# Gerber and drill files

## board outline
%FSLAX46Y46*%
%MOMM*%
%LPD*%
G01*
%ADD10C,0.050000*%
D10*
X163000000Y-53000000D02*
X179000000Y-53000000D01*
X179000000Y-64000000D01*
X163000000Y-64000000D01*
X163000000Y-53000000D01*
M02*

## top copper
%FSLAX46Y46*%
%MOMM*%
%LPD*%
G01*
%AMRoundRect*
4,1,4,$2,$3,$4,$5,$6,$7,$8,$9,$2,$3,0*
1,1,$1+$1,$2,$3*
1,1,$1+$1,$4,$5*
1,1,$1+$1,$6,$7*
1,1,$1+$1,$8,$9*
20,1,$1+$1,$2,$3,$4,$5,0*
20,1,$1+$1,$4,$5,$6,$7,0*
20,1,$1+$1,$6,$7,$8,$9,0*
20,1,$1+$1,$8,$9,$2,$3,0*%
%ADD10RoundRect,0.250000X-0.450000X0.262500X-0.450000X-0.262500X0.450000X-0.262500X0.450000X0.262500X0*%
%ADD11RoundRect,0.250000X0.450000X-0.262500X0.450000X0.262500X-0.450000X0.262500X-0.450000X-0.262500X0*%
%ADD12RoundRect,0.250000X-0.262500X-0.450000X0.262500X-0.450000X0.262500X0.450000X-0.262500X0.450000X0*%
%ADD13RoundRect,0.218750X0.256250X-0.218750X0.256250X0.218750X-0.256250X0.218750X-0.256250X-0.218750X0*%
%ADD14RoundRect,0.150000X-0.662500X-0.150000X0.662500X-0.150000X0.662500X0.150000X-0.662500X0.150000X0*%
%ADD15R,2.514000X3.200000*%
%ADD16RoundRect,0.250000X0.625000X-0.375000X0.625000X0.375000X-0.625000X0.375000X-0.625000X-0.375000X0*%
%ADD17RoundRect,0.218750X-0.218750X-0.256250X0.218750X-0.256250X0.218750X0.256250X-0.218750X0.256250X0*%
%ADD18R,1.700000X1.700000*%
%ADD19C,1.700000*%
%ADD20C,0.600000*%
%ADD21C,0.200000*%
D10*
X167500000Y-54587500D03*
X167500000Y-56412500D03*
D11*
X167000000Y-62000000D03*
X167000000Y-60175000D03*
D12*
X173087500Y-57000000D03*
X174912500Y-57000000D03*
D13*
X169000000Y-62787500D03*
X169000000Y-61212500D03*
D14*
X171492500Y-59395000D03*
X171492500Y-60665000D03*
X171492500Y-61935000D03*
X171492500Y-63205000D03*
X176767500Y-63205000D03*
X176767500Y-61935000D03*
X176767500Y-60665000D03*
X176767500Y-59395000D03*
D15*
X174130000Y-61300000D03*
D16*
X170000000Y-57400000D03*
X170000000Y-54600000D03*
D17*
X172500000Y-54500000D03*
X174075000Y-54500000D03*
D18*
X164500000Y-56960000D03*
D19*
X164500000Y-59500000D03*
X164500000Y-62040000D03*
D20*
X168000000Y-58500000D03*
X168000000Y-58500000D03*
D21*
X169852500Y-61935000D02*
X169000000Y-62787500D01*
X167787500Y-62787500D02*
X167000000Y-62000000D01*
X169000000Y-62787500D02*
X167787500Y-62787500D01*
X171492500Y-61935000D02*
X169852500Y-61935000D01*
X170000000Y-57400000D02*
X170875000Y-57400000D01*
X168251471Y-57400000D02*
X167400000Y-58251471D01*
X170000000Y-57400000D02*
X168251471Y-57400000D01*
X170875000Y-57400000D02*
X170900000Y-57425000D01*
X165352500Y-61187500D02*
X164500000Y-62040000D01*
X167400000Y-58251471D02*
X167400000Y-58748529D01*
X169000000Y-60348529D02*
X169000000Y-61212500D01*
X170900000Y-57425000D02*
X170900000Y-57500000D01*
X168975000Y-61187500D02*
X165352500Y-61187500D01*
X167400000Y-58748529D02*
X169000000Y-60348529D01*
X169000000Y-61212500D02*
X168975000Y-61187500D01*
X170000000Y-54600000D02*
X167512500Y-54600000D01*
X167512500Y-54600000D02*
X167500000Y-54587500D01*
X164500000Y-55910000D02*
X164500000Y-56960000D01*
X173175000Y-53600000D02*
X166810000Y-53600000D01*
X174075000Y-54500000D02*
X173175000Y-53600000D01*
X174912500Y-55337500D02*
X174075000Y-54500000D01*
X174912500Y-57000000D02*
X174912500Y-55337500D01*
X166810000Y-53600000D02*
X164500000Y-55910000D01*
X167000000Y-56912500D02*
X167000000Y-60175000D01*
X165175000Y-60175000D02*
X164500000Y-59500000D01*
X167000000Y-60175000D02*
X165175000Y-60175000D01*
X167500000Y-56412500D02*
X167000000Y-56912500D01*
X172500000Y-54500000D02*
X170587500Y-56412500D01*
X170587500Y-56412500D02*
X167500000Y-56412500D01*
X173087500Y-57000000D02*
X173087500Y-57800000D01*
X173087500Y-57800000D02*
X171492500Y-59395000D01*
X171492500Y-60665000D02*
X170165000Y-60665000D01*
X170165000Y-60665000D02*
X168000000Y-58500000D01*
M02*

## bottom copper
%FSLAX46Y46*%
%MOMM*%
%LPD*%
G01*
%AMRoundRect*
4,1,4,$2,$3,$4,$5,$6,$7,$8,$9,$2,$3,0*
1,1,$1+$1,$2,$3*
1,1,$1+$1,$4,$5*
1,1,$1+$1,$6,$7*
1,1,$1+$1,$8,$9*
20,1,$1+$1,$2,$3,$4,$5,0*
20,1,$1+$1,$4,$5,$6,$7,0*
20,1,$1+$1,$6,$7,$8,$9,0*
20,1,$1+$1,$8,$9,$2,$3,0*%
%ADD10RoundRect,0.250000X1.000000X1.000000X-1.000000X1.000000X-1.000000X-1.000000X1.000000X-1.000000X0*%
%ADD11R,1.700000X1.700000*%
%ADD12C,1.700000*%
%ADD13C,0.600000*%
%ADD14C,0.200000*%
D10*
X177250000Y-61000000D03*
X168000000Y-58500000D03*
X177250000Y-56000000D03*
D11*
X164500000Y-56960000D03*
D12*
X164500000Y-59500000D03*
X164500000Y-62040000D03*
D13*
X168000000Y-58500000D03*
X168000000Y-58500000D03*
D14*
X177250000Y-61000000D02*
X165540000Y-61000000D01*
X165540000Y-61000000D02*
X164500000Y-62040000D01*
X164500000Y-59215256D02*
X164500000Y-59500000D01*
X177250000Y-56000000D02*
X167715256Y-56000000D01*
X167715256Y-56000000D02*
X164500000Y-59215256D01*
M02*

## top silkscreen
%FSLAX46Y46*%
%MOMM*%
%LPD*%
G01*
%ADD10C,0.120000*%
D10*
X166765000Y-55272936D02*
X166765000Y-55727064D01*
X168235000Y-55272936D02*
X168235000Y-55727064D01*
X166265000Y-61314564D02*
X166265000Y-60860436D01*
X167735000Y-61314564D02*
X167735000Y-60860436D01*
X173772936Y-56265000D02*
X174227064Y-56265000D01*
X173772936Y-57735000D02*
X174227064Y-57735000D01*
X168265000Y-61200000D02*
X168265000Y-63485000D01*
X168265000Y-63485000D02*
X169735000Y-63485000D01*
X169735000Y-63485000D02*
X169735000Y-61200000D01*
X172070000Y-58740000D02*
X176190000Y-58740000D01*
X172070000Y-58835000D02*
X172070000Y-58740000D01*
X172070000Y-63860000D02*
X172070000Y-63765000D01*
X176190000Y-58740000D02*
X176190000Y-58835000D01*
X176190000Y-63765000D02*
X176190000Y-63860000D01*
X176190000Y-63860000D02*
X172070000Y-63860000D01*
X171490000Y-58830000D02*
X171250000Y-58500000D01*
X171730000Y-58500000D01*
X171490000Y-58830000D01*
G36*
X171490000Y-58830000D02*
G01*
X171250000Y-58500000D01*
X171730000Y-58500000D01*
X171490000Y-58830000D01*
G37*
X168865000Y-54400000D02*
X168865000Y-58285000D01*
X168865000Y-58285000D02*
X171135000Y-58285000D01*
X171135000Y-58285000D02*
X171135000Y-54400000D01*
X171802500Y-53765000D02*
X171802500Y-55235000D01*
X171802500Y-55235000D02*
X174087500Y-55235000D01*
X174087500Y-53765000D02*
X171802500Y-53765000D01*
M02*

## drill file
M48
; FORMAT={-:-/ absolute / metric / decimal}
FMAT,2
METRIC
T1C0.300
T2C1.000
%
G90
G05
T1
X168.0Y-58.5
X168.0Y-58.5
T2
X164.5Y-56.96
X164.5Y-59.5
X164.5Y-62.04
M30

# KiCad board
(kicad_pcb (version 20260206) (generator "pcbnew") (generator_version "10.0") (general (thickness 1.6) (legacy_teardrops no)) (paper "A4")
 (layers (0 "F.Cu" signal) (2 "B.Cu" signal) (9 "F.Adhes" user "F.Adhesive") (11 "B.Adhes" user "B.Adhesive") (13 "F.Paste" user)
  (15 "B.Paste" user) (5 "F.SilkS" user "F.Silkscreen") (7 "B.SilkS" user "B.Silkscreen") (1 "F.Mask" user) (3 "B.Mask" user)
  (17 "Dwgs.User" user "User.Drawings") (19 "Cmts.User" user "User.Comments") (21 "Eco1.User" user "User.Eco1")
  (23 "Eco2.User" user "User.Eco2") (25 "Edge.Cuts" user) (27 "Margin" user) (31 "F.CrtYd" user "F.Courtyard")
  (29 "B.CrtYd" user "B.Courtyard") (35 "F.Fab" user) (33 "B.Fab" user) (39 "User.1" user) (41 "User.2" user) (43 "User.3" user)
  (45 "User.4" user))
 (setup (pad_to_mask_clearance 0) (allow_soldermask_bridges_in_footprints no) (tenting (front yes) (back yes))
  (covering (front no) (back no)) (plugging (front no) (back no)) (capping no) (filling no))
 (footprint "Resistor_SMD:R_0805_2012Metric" (layer "F.Cu") (at 167.5 55.5 -90)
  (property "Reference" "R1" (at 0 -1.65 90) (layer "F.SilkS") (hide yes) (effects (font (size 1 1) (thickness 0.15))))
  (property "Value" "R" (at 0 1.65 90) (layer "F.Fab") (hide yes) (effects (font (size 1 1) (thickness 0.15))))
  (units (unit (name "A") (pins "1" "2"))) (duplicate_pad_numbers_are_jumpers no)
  (fp_line (start -0.227064 0.735) (end 0.227064 0.735) (stroke (width 0.12) (type solid)) (layer "F.SilkS"))
  (fp_line (start -0.227064 -0.735) (end 0.227064 -0.735) (stroke (width 0.12) (type solid)) (layer "F.SilkS"))
  (pad "1" smd roundrect (at -0.9125 0 270) (size 1.025 1.4) (layers "F.Cu" "F.Mask" "F.Paste") (roundrect_rratio 0.243902)
   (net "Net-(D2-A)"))
  (pad "2" smd roundrect (at 0.9125 0 270) (size 1.025 1.4) (layers "F.Cu" "F.Mask" "F.Paste") (roundrect_rratio 0.243902) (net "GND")))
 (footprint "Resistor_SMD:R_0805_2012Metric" (layer "F.Cu") (at 167 61.0875 90)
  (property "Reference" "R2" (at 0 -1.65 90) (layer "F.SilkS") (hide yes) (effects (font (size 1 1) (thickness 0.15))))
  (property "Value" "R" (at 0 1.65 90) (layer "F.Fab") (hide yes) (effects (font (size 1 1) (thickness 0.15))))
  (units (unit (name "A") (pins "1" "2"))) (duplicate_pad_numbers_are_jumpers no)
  (fp_line (start -0.227064 -0.735) (end 0.227064 -0.735) (stroke (width 0.12) (type solid)) (layer "F.SilkS"))
  (fp_line (start -0.227064 0.735) (end 0.227064 0.735) (stroke (width 0.12) (type solid)) (layer "F.SilkS"))
  (pad "1" smd roundrect (at -0.9125 0 90) (size 1.025 1.4) (layers "F.Cu" "F.Mask" "F.Paste") (roundrect_rratio 0.243902)
   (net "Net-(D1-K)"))
  (pad "2" smd roundrect (at 0.9125 0 90) (size 1.025 1.4) (layers "F.Cu" "F.Mask" "F.Paste") (roundrect_rratio 0.243902) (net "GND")))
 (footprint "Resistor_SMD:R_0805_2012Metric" (layer "F.Cu") (at 174 57)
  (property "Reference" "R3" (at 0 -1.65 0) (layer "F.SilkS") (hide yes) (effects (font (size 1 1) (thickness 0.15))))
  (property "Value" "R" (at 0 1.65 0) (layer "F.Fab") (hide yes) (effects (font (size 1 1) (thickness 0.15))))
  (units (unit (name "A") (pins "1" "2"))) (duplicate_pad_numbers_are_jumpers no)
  (fp_line (start -0.227064 -0.735) (end 0.227064 -0.735) (stroke (width 0.12) (type solid)) (layer "F.SilkS"))
  (fp_line (start -0.227064 0.735) (end 0.227064 0.735) (stroke (width 0.12) (type solid)) (layer "F.SilkS"))
  (pad "1" smd roundrect (at -0.9125 0) (size 1.025 1.4) (layers "F.Cu" "F.Mask" "F.Paste") (roundrect_rratio 0.243902)
   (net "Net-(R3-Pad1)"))
  (pad "2" smd roundrect (at 0.9125 0) (size 1.025 1.4) (layers "F.Cu" "F.Mask" "F.Paste") (roundrect_rratio 0.243902) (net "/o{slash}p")))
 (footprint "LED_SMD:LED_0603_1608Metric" (layer "F.Cu") (at 169 62 90)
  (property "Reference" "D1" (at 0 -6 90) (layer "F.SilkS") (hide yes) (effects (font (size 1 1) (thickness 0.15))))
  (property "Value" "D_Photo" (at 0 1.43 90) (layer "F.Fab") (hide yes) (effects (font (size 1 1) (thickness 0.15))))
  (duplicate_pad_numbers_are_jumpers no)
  (fp_line (start 0.8 -0.735) (end -1.485 -0.735) (stroke (width 0.12) (type solid)) (layer "F.SilkS"))
  (fp_line (start -1.485 -0.735) (end -1.485 0.735) (stroke (width 0.12) (type solid)) (layer "F.SilkS"))
  (fp_line (start -1.485 0.735) (end 0.8 0.735) (stroke (width 0.12) (type solid)) (layer "F.SilkS"))
  (pad "1" smd roundrect (at -0.7875 0 90) (size 0.875 0.95) (layers "F.Cu" "F.Mask" "F.Paste") (roundrect_rratio 0.25) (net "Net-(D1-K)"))
  (pad "2" smd roundrect (at 0.7875 0 90) (size 0.875 0.95) (layers "F.Cu" "F.Mask" "F.Paste") (roundrect_rratio 0.25) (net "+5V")))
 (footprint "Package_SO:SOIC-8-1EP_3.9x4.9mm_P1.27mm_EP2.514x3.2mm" (layer "F.Cu") (at 174.13 61.3)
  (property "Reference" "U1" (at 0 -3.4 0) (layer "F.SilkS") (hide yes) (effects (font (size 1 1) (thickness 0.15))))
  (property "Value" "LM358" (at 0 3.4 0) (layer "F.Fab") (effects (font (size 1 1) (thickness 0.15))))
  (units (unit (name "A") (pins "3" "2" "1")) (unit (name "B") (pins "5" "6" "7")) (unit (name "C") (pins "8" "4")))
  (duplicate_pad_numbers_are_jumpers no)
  (fp_line (start -2.06 -2.56) (end 2.06 -2.56) (stroke (width 0.12) (type solid)) (layer "F.SilkS"))
  (fp_line (start -2.06 -2.465) (end -2.06 -2.56) (stroke (width 0.12) (type solid)) (layer "F.SilkS"))
  (fp_line (start -2.06 2.56) (end -2.06 2.465) (stroke (width 0.12) (type solid)) (layer "F.SilkS"))
  (fp_line (start 2.06 -2.56) (end 2.06 -2.465) (stroke (width 0.12) (type solid)) (layer "F.SilkS"))
  (fp_line (start 2.06 2.465) (end 2.06 2.56) (stroke (width 0.12) (type solid)) (layer "F.SilkS"))
  (fp_line (start 2.06 2.56) (end -2.06 2.56) (stroke (width 0.12) (type solid)) (layer "F.SilkS"))
  (fp_poly (pts (xy -2.64 -2.47) (xy -2.88 -2.8) (xy -2.4 -2.8)) (stroke (width 0.12) (type solid)) (fill yes) (layer "F.SilkS"))
  (pad "" smd roundrect (at -0.63 -0.8) (size 1.01 1.29) (layers "F.Paste") (roundrect_rratio 0.247525))
  (pad "" smd roundrect (at -0.63 0.8) (size 1.01 1.29) (layers "F.Paste") (roundrect_rratio 0.247525))
  (pad "" smd roundrect (at 0.63 -0.8) (size 1.01 1.29) (layers "F.Paste") (roundrect_rratio 0.247525))
  (pad "" smd roundrect (at 0.63 0.8) (size 1.01 1.29) (layers "F.Paste") (roundrect_rratio 0.247525))
  (pad "1" smd roundrect (at -2.6375 -1.905) (size 1.625 0.6) (layers "F.Cu" "F.Mask" "F.Paste") (roundrect_rratio 0.25)
   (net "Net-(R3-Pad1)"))
  (pad "2" smd roundrect (at -2.6375 -0.635) (size 1.625 0.6) (layers "F.Cu" "F.Mask" "F.Paste") (roundrect_rratio 0.25) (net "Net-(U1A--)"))
  (pad "3" smd roundrect (at -2.6375 0.635) (size 1.625 0.6) (layers "F.Cu" "F.Mask" "F.Paste") (roundrect_rratio 0.25) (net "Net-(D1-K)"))
  (pad "4" smd roundrect (at -2.6375 1.905) (size 1.625 0.6) (layers "F.Cu" "F.Mask" "F.Paste") (roundrect_rratio 0.25))
  (pad "5" smd roundrect (at 2.6375 1.905) (size 1.625 0.6) (layers "F.Cu" "F.Mask" "F.Paste") (roundrect_rratio 0.25))
  (pad "6" smd roundrect (at 2.6375 0.635) (size 1.625 0.6) (layers "F.Cu" "F.Mask" "F.Paste") (roundrect_rratio 0.25))
  (pad "7" smd roundrect (at 2.6375 -0.635) (size 1.625 0.6) (layers "F.Cu" "F.Mask" "F.Paste") (roundrect_rratio 0.25))
  (pad "8" smd roundrect (at 2.6375 -1.905) (size 1.625 0.6) (layers "F.Cu" "F.Mask" "F.Paste") (roundrect_rratio 0.25))
  (pad "9" smd rect (at 0 0) (size 2.514 3.2) (layers "F.Cu" "F.Mask") (zone_connect 2)))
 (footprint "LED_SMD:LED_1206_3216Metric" (layer "F.Cu") (at 170 56 90)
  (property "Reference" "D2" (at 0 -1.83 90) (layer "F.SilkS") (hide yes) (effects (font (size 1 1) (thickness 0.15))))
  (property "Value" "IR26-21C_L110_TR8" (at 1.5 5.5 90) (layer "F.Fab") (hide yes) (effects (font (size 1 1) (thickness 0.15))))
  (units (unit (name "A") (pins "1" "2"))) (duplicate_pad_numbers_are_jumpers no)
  (fp_line (start 1.6 -1.135) (end -2.285 -1.135) (stroke (width 0.12) (type solid)) (layer "F.SilkS"))
  (fp_line (start -2.285 -1.135) (end -2.285 1.135) (stroke (width 0.12) (type solid)) (layer "F.SilkS"))
  (fp_line (start -2.285 1.135) (end 1.6 1.135) (stroke (width 0.12) (type solid)) (layer "F.SilkS"))
  (pad "1" smd roundrect (at -1.4 0 90) (size 1.25 1.75) (layers "F.Cu" "F.Mask" "F.Paste") (roundrect_rratio 0.2) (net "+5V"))
  (pad "2" smd roundrect (at 1.4 0 90) (size 1.25 1.75) (layers "F.Cu" "F.Mask" "F.Paste") (roundrect_rratio 0.2) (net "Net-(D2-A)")))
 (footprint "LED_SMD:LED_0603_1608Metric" (layer "F.Cu") (at 173.2875 54.5)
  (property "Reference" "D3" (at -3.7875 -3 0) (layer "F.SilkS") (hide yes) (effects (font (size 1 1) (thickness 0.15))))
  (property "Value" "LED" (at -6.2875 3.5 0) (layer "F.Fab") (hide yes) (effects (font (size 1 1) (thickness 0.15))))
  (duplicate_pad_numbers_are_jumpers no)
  (fp_line (start -1.485 -0.735) (end -1.485 0.735) (stroke (width 0.12) (type solid)) (layer "F.SilkS"))
  (fp_line (start -1.485 0.735) (end 0.8 0.735) (stroke (width 0.12) (type solid)) (layer "F.SilkS"))
  (fp_line (start 0.8 -0.735) (end -1.485 -0.735) (stroke (width 0.12) (type solid)) (layer "F.SilkS"))
  (pad "1" smd roundrect (at -0.7875 0) (size 0.875 0.95) (layers "F.Cu" "F.Mask" "F.Paste") (roundrect_rratio 0.25) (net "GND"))
  (pad "2" smd roundrect (at 0.7875 0) (size 0.875 0.95) (layers "F.Cu" "F.Mask" "F.Paste") (roundrect_rratio 0.25) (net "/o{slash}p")))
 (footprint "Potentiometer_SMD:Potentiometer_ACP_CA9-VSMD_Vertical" (layer "B.Cu") (at 172.625 58.5 180)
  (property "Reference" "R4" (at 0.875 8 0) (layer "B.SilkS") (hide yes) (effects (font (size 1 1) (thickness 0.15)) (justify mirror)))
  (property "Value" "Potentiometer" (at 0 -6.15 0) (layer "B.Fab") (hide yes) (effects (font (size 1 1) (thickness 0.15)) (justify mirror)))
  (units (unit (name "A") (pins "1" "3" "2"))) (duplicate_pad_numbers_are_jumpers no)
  (pad "1" smd roundrect (at -4.625 -2.5 180) (size 2.5 2.5) (layers "B.Cu" "B.Mask" "B.Paste") (roundrect_rratio 0.1) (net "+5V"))
  (pad "2" smd roundrect (at 4.625 0 180) (size 2.5 2.5) (layers "B.Cu" "B.Mask" "B.Paste") (roundrect_rratio 0.1) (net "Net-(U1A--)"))
  (pad "3" smd roundrect (at -4.625 2.5 180) (size 2.5 2.5) (layers "B.Cu" "B.Mask" "B.Paste") (roundrect_rratio 0.1) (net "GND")))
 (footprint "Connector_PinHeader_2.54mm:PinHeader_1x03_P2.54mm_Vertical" (layer "B.Cu") (at 164.5 56.96 180)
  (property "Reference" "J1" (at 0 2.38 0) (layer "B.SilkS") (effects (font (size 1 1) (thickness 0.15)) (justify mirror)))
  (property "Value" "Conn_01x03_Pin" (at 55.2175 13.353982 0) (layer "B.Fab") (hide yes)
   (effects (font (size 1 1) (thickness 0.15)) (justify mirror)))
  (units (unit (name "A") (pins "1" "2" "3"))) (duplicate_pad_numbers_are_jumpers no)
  (pad "1" thru_hole rect (at 0 0 180) (size 1.7 1.7) (drill 1) (layers "*.Cu" "*.Mask") (remove_unused_layers no) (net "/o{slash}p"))
  (pad "2" thru_hole circle (at 0 -2.54 180) (size 1.7 1.7) (drill 1) (layers "*.Cu" "*.Mask") (remove_unused_layers no) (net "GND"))
  (pad "3" thru_hole circle (at 0 -5.08 180) (size 1.7 1.7) (drill 1) (layers "*.Cu" "*.Mask") (remove_unused_layers no) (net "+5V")))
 (gr_rect (start 163 53) (end 179 64) (stroke (width 0.05) (type default)) (fill no) (layer "Edge.Cuts"))
 (segment (start 169.8525 61.935) (end 169 62.7875) (width 0.2) (layer "F.Cu") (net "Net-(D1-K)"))
 (segment (start 167.7875 62.7875) (end 167 62) (width 0.2) (layer "F.Cu") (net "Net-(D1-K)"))
 (segment (start 169 62.7875) (end 167.7875 62.7875) (width 0.2) (layer "F.Cu") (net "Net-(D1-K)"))
 (segment (start 171.4925 61.935) (end 169.8525 61.935) (width 0.2) (layer "F.Cu") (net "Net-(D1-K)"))
 (segment (start 170 57.4) (end 170.875 57.4) (width 0.2) (layer "F.Cu") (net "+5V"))
 (segment (start 168.251471 57.4) (end 167.4 58.251471) (width 0.2) (layer "F.Cu") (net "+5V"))
 (segment (start 170 57.4) (end 168.251471 57.4) (width 0.2) (layer "F.Cu") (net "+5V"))
 (segment (start 170.875 57.4) (end 170.9 57.425) (width 0.2) (layer "F.Cu") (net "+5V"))
 (segment (start 165.3525 61.1875) (end 164.5 62.04) (width 0.2) (layer "F.Cu") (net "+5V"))
 (segment (start 167.4 58.251471) (end 167.4 58.748529) (width 0.2) (layer "F.Cu") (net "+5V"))
 (segment (start 169 60.348529) (end 169 61.2125) (width 0.2) (layer "F.Cu") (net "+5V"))
 (segment (start 170.9 57.425) (end 170.9 57.5) (width 0.2) (layer "F.Cu") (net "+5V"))
 (segment (start 168.975 61.1875) (end 165.3525 61.1875) (width 0.2) (layer "F.Cu") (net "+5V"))
 (segment (start 167.4 58.748529) (end 169 60.348529) (width 0.2) (layer "F.Cu") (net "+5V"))
 (segment (start 169 61.2125) (end 168.975 61.1875) (width 0.2) (layer "F.Cu") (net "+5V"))
 (segment (start 177.25 61) (end 165.54 61) (width 0.2) (layer "B.Cu") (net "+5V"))
 (segment (start 165.54 61) (end 164.5 62.04) (width 0.2) (layer "B.Cu") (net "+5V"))
 (segment (start 170 54.6) (end 167.5125 54.6) (width 0.2) (layer "F.Cu") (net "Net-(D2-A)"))
 (segment (start 167.5125 54.6) (end 167.5 54.5875) (width 0.2) (layer "F.Cu") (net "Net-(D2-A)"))
 (segment (start 164.5 55.91) (end 164.5 56.96) (width 0.2) (layer "F.Cu") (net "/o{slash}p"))
 (segment (start 173.175 53.6) (end 166.81 53.6) (width 0.2) (layer "F.Cu") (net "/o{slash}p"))
 (segment (start 174.075 54.5) (end 173.175 53.6) (width 0.2) (layer "F.Cu") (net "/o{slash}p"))
 (segment (start 174.9125 55.3375) (end 174.075 54.5) (width 0.2) (layer "F.Cu") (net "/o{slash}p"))
 (segment (start 174.9125 57) (end 174.9125 55.3375) (width 0.2) (layer "F.Cu") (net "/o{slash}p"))
 (segment (start 166.81 53.6) (end 164.5 55.91) (width 0.2) (layer "F.Cu") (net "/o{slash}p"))
 (segment (start 167 56.9125) (end 167 60.175) (width 0.2) (layer "F.Cu") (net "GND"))
 (segment (start 165.175 60.175) (end 164.5 59.5) (width 0.2) (layer "F.Cu") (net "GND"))
 (segment (start 167 60.175) (end 165.175 60.175) (width 0.2) (layer "F.Cu") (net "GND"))
 (segment (start 167.5 56.4125) (end 167 56.9125) (width 0.2) (layer "F.Cu") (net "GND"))
 (segment (start 172.5 54.5) (end 170.5875 56.4125) (width 0.2) (layer "F.Cu") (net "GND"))
 (segment (start 170.5875 56.4125) (end 167.5 56.4125) (width 0.2) (layer "F.Cu") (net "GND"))
 (segment (start 164.5 59.215256) (end 164.5 59.5) (width 0.2) (layer "B.Cu") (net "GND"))
 (segment (start 177.25 56) (end 167.715256 56) (width 0.2) (layer "B.Cu") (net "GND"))
 (segment (start 167.715256 56) (end 164.5 59.215256) (width 0.2) (layer "B.Cu") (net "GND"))
 (segment (start 173.0875 57) (end 173.0875 57.8) (width 0.2) (layer "F.Cu") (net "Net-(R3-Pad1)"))
 (segment (start 173.0875 57.8) (end 171.4925 59.395) (width 0.2) (layer "F.Cu") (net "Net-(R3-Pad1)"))
 (segment (start 171.4925 60.665) (end 170.165 60.665) (width 0.2) (layer "F.Cu") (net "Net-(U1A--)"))
 (segment (start 170.165 60.665) (end 168 58.5) (width 0.2) (layer "F.Cu") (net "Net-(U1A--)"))
 (via (at 168 58.5) (size 0.6) (drill 0.3) (layers "F.Cu" "B.Cu") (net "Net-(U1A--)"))
 (via (at 168 58.5) (size 0.6) (drill 0.3) (layers "F.Cu" "B.Cu") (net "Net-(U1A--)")))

